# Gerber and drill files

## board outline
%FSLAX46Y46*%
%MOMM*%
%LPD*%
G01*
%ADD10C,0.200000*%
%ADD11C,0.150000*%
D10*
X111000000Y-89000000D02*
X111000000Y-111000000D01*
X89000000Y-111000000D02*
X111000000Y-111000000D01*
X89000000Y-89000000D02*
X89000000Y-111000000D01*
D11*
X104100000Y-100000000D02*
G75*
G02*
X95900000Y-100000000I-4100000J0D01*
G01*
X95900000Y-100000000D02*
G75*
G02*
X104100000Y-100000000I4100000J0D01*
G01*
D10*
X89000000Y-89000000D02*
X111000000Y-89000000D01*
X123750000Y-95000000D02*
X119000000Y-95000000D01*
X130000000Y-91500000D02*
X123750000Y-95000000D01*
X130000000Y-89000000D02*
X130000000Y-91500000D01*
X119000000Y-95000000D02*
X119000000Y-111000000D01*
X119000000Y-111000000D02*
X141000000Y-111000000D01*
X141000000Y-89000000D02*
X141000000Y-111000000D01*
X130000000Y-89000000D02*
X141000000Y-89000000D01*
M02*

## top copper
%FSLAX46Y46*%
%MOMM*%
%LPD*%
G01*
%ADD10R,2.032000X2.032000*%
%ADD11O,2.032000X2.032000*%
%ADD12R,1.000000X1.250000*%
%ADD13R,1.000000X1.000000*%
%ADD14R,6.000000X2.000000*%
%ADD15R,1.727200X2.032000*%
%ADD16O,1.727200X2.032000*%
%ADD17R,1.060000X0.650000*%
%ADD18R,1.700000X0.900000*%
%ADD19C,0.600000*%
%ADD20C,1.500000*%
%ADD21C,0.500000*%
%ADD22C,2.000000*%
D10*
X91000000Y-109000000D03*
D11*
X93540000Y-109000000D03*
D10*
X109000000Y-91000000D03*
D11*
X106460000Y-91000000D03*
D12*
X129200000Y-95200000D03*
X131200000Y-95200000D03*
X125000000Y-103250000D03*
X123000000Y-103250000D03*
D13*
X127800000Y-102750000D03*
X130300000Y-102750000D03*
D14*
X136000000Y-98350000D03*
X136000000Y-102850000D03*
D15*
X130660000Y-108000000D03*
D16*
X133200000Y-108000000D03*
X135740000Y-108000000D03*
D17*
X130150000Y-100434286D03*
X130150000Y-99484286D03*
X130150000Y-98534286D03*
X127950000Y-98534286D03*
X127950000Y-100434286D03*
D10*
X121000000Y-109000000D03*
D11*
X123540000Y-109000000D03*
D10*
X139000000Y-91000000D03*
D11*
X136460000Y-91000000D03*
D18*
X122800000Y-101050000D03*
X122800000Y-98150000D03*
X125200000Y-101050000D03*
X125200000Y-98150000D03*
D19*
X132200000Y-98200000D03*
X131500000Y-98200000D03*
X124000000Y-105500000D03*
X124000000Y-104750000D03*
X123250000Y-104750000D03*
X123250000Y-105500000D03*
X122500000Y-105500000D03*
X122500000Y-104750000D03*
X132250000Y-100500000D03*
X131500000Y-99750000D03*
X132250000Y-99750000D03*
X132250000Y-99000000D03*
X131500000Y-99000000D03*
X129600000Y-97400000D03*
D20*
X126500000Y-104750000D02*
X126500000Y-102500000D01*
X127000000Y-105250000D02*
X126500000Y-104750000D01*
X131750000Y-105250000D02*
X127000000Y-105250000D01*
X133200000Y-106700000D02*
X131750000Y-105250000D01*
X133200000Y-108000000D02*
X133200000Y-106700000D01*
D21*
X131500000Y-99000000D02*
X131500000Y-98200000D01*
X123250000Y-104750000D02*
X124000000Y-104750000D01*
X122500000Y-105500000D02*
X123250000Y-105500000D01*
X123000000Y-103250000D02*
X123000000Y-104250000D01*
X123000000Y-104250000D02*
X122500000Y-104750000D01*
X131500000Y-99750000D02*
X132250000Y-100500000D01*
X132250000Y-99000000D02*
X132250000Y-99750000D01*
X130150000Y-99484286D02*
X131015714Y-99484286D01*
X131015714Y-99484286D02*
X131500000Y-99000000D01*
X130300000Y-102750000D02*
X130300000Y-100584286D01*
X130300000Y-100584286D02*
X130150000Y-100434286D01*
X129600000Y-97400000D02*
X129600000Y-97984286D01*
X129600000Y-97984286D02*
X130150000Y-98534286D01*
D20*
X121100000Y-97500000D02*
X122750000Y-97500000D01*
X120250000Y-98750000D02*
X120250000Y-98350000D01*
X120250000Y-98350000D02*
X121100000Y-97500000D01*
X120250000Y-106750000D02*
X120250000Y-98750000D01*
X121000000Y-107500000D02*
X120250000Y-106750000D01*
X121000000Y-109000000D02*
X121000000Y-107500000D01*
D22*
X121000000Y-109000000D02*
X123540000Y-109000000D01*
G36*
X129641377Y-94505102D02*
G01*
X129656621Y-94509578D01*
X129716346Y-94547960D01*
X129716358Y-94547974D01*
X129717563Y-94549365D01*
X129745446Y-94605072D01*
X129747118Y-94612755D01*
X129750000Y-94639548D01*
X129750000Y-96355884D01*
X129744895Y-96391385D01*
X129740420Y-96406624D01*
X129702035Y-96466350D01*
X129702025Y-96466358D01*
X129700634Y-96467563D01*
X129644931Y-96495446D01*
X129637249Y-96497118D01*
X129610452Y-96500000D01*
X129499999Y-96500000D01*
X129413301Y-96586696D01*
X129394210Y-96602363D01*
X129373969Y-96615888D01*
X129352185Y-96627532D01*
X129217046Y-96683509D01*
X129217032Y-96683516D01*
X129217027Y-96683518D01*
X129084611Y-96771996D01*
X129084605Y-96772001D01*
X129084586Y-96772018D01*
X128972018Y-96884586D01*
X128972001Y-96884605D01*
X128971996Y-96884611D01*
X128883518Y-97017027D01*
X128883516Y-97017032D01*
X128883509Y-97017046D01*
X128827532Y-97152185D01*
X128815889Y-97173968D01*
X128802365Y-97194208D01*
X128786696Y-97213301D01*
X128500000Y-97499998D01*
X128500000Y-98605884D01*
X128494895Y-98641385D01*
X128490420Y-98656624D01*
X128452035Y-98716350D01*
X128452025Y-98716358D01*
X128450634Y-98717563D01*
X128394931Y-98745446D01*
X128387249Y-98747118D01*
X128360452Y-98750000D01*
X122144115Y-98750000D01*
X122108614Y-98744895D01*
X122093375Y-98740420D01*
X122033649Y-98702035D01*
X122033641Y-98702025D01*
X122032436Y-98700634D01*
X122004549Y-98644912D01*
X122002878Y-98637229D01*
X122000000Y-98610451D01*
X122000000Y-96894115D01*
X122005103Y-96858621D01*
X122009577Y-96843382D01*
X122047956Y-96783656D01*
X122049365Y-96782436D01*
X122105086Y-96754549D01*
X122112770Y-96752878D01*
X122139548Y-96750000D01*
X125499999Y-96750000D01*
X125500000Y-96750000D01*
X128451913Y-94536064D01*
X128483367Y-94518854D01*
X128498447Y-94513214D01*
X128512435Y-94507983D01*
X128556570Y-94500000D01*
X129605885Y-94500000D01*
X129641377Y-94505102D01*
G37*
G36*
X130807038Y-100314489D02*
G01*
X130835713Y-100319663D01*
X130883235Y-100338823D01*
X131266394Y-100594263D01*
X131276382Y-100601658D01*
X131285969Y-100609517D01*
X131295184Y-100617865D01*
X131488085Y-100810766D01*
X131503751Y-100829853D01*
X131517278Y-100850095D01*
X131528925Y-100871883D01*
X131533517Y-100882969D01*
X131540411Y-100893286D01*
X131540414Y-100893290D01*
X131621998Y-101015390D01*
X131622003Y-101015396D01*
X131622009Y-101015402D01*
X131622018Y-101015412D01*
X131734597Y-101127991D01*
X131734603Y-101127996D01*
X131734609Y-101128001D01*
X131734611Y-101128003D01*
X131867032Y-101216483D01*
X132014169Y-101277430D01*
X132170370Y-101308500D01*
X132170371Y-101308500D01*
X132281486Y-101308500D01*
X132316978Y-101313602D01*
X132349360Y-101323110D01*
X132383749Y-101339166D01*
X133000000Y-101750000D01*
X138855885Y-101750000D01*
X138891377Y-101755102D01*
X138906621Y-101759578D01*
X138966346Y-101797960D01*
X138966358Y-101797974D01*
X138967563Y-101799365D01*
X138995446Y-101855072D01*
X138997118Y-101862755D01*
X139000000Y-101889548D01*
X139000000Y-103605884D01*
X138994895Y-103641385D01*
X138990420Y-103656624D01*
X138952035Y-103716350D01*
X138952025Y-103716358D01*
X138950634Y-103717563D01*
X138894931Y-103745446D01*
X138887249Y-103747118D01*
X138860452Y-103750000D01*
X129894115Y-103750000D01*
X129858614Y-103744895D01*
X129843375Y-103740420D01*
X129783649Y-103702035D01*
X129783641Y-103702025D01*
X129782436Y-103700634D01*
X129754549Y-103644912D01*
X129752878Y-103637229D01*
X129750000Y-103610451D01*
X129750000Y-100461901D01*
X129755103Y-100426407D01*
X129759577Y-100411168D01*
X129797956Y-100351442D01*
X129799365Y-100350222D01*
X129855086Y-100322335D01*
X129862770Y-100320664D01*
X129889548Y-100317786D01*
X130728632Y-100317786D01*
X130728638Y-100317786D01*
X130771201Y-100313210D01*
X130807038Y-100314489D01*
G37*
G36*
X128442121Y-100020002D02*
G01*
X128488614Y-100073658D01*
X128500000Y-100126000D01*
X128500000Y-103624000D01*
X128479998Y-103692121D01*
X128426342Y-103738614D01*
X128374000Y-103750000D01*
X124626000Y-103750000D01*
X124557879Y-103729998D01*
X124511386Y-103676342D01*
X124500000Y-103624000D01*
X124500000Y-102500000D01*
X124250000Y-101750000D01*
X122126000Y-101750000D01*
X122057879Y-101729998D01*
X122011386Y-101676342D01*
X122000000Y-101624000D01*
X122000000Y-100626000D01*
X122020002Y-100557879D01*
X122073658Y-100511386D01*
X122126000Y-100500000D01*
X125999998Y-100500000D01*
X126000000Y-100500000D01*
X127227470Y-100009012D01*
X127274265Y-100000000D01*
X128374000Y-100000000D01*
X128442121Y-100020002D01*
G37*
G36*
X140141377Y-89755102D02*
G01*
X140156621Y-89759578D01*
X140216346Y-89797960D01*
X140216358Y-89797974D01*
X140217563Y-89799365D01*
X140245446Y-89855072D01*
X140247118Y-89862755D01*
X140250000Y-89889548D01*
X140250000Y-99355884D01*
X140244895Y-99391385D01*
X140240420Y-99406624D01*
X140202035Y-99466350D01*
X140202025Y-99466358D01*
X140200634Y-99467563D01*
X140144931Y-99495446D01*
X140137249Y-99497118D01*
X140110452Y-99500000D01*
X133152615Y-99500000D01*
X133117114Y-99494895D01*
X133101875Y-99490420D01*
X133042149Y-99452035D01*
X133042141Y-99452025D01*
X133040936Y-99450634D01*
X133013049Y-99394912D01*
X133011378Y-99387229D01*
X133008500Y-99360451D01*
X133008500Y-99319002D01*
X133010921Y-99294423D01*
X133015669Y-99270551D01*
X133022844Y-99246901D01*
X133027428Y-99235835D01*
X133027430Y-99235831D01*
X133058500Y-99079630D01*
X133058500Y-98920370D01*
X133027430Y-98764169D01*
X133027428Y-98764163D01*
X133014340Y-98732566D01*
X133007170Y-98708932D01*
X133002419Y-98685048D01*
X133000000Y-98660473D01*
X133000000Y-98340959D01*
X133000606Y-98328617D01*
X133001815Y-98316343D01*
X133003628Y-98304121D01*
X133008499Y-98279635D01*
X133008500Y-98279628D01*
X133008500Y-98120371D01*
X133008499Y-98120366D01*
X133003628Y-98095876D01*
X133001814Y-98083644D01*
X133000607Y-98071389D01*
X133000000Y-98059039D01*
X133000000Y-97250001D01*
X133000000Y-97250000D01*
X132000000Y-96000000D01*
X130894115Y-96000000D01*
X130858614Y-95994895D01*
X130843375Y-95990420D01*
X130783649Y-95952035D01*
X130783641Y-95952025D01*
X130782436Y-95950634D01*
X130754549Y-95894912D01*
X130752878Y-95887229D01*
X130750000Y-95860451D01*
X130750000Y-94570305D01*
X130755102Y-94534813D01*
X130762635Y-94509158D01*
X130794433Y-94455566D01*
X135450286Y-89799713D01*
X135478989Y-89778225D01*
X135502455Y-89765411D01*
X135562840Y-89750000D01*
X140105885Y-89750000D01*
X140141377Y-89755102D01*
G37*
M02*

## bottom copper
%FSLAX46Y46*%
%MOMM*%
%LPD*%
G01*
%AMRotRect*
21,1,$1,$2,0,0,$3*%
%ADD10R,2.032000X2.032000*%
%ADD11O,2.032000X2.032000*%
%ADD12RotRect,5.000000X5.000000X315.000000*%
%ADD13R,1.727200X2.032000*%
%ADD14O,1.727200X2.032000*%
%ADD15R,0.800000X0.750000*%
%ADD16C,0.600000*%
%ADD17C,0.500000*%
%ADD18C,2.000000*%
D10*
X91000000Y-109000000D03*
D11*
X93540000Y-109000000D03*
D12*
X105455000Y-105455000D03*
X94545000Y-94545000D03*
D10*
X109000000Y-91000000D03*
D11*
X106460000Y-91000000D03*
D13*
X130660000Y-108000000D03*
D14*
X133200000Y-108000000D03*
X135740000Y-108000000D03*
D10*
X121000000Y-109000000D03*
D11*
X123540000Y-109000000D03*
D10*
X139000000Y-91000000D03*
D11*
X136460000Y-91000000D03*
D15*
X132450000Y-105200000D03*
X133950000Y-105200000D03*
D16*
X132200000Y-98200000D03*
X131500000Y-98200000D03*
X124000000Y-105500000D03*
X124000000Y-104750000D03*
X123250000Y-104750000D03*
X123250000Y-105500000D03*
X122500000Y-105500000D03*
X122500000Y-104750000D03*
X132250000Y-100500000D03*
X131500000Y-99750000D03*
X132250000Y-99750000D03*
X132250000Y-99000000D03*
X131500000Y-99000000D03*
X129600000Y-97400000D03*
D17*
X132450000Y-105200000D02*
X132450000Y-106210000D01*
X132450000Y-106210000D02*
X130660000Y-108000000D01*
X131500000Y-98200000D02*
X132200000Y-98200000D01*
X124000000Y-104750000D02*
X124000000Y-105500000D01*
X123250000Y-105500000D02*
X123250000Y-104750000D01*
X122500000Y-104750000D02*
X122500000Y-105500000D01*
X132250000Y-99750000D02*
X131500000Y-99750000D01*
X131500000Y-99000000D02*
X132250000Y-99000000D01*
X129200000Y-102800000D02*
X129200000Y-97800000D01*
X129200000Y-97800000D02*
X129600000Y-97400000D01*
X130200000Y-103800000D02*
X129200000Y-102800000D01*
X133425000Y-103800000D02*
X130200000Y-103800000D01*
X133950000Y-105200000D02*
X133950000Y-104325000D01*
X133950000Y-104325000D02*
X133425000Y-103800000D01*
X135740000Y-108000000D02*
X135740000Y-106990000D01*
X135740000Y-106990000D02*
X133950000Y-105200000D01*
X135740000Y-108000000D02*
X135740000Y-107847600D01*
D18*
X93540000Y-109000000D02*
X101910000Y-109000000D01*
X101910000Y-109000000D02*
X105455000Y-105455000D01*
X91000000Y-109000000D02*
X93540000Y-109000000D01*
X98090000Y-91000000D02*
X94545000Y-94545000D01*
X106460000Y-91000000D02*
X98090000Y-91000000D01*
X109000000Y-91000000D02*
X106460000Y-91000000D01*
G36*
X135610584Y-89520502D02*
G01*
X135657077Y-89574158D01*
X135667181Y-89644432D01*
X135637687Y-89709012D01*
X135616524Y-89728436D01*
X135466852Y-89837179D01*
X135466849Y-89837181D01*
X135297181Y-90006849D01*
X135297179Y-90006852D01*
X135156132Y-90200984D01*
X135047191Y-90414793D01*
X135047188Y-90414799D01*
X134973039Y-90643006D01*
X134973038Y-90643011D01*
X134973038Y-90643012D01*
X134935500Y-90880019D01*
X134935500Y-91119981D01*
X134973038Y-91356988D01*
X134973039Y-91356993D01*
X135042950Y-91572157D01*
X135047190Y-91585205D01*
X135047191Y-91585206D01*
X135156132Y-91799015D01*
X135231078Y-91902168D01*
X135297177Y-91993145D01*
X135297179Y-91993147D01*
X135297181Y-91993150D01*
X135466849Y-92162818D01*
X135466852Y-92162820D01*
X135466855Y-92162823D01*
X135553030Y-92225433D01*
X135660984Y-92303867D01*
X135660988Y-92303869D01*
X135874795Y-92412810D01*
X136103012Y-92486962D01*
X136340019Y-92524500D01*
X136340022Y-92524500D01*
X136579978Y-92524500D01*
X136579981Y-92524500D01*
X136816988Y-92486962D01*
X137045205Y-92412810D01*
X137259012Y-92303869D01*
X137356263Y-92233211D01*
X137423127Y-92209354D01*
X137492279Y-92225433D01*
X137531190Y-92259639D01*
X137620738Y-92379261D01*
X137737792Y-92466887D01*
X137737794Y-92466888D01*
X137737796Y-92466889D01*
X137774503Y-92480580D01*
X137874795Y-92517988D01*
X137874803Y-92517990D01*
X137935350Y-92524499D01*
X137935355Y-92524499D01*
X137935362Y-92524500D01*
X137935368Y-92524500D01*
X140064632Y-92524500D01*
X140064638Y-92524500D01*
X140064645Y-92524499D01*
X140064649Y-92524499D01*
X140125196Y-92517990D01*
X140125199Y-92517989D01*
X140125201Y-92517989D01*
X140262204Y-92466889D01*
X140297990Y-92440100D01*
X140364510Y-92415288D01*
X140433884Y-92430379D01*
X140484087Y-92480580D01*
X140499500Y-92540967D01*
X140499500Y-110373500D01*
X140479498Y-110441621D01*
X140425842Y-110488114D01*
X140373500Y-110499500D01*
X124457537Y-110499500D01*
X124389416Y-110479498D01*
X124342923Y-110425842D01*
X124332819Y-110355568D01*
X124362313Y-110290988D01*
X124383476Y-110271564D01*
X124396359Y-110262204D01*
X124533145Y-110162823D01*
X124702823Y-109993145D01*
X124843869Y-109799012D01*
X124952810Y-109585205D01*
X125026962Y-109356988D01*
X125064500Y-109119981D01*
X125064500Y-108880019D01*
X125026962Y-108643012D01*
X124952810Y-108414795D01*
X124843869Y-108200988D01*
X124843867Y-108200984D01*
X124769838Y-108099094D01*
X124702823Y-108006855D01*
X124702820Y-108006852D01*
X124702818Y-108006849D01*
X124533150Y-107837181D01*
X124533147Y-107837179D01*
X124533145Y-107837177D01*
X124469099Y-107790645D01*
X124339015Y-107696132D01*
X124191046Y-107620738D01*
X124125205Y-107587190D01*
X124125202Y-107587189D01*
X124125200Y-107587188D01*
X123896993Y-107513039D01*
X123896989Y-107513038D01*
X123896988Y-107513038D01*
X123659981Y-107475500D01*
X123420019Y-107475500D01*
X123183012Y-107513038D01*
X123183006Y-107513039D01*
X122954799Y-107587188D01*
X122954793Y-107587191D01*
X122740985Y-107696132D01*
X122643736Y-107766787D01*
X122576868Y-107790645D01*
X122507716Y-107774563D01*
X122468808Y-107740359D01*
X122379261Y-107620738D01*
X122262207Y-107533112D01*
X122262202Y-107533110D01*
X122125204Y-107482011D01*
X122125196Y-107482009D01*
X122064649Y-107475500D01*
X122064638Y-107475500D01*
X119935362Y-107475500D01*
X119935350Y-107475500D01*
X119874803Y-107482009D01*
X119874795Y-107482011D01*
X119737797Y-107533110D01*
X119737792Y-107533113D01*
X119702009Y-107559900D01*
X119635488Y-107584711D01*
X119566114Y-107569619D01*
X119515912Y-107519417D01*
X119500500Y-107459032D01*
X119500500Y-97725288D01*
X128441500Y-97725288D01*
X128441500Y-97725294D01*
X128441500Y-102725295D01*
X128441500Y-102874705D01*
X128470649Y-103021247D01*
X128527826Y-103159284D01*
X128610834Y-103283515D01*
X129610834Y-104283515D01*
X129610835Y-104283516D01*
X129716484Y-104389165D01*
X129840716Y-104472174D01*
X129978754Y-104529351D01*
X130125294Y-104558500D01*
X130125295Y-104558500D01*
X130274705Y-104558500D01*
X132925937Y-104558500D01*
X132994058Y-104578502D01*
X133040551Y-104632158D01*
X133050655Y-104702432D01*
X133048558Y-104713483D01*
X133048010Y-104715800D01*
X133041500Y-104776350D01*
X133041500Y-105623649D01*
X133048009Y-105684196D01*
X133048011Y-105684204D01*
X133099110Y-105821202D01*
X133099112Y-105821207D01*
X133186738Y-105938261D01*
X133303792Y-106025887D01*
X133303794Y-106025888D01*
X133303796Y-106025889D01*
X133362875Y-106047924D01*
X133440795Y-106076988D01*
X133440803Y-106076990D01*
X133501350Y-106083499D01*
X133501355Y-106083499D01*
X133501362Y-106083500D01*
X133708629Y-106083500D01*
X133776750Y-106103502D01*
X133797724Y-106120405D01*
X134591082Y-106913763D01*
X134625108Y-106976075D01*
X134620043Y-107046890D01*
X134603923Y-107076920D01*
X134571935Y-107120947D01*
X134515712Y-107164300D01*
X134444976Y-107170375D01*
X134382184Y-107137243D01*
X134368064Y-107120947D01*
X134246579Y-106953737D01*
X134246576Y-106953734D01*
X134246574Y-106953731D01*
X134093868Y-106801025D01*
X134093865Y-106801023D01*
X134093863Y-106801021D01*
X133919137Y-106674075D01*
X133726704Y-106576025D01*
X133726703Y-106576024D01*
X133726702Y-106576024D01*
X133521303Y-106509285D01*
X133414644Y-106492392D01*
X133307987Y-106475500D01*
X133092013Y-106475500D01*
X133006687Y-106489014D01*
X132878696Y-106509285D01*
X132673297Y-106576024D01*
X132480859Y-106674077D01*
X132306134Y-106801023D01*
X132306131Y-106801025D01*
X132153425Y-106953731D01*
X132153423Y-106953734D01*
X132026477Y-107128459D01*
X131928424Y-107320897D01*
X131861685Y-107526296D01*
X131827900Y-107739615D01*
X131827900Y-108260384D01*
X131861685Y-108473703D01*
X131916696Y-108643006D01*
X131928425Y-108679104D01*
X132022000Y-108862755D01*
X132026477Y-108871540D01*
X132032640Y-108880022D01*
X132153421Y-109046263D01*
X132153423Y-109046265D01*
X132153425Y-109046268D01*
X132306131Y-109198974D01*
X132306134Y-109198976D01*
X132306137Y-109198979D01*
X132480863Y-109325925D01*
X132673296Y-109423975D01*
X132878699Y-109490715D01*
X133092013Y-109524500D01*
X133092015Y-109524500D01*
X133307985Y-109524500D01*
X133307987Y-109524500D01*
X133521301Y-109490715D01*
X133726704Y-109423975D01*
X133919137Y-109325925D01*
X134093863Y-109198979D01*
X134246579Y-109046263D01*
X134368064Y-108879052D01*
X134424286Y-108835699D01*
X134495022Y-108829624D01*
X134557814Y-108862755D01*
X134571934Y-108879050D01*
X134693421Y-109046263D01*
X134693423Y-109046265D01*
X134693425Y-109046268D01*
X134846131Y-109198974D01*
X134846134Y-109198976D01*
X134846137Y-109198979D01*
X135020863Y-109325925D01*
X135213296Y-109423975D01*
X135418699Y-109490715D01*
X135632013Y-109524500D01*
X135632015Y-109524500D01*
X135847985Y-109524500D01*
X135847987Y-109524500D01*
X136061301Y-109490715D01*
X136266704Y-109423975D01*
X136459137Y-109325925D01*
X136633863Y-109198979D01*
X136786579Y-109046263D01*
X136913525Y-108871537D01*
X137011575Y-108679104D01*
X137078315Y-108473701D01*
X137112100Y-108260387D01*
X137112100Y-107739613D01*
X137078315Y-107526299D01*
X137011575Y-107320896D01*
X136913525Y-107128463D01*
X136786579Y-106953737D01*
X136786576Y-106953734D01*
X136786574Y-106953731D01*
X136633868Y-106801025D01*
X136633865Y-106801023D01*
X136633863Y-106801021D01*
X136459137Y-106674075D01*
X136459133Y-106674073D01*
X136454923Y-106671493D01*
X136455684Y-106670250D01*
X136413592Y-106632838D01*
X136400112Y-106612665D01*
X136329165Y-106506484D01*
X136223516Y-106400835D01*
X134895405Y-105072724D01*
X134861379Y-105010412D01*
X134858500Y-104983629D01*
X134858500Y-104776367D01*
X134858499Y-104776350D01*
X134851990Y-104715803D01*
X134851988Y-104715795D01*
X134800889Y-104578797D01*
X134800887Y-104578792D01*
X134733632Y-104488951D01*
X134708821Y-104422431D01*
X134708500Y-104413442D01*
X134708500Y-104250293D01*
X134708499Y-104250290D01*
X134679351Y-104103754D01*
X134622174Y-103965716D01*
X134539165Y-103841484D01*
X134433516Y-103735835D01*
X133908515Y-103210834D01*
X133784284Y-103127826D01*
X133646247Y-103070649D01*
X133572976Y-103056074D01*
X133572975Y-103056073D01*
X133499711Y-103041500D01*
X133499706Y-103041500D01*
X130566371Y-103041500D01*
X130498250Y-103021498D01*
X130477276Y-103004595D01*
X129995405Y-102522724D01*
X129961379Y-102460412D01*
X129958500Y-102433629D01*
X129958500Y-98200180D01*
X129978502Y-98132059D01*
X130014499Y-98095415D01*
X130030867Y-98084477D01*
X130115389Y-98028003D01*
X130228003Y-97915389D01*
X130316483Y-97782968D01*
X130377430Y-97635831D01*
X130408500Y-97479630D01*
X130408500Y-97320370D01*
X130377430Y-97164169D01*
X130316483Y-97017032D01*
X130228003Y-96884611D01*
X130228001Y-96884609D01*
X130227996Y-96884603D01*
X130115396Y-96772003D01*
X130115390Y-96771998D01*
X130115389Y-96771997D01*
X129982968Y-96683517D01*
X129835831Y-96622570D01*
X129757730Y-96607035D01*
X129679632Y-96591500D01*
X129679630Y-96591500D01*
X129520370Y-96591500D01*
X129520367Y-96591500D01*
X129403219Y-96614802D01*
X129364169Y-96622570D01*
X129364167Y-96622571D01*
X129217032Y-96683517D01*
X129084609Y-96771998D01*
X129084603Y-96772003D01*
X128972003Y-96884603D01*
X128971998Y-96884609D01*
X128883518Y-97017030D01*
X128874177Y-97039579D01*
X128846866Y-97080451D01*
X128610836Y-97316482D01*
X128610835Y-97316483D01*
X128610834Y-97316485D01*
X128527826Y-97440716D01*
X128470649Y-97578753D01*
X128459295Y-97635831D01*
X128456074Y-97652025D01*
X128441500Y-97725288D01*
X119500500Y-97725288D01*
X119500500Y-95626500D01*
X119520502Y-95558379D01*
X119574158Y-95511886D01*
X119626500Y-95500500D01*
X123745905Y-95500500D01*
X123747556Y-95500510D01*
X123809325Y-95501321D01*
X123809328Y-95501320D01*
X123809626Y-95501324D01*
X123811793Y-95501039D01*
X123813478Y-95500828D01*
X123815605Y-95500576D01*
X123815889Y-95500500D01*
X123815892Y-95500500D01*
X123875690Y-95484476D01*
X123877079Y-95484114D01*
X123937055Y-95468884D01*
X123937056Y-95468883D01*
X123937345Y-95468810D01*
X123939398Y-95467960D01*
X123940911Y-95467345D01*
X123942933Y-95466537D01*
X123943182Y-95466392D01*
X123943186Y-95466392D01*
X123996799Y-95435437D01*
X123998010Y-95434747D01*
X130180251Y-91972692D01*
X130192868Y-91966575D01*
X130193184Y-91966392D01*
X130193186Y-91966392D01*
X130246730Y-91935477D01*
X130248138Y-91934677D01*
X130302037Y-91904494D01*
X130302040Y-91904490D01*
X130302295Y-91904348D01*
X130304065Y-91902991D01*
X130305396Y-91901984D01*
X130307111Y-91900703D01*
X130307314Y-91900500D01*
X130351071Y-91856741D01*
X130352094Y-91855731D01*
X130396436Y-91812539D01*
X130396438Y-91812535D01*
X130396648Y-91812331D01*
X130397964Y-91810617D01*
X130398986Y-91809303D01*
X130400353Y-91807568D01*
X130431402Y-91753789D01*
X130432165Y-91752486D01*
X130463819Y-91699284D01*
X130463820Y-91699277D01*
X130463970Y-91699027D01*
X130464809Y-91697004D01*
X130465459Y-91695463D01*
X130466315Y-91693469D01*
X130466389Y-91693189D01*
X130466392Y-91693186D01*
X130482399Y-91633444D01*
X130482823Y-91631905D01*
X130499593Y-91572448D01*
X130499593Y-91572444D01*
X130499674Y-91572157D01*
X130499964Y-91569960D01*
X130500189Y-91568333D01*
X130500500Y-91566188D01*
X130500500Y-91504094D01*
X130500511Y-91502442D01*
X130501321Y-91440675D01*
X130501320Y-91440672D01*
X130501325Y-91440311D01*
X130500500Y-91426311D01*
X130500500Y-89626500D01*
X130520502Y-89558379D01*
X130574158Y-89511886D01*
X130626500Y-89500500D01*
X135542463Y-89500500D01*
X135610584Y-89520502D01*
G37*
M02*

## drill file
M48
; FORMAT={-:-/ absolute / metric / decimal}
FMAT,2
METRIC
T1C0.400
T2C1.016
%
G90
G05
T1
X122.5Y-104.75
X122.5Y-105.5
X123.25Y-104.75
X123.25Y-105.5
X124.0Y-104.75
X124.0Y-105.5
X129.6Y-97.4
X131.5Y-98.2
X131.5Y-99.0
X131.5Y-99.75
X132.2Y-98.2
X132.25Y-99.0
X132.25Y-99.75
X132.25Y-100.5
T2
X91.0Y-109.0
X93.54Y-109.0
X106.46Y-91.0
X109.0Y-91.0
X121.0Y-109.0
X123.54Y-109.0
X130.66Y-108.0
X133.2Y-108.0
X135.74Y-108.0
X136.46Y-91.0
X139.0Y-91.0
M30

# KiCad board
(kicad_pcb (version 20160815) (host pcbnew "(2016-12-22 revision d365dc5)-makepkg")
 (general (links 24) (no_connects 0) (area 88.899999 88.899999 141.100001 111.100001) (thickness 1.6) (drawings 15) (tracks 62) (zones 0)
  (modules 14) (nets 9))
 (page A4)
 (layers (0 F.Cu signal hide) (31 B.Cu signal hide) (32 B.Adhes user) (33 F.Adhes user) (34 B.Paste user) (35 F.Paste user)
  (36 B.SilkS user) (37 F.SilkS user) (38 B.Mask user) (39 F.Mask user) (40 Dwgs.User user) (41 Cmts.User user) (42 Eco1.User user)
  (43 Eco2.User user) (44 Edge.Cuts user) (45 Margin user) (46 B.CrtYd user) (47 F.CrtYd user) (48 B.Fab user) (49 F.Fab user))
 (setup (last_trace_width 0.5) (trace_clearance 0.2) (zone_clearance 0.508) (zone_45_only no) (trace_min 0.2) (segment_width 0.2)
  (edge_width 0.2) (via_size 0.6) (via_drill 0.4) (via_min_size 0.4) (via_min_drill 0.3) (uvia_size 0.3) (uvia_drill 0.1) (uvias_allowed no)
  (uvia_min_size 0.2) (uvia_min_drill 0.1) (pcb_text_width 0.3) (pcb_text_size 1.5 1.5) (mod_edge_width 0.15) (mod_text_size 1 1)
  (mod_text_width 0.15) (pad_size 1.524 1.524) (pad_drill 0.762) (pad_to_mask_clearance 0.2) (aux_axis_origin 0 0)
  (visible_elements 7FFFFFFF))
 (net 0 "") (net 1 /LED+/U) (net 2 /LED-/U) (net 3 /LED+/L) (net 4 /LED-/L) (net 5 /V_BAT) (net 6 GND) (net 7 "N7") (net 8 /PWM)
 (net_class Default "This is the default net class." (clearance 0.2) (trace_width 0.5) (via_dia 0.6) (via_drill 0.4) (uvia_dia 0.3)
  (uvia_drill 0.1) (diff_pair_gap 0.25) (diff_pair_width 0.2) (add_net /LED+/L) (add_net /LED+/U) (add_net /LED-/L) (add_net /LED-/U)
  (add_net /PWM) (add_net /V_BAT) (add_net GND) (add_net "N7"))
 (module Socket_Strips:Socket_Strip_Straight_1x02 (layer B.Cu) (at 91 109)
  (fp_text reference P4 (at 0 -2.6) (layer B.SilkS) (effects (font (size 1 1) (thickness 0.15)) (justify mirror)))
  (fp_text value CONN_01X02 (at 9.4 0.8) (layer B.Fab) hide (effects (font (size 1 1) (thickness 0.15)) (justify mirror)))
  (pad 1 thru_hole rect (at 0 0) (size 2.032 2.032) (drill 1.016) (layers *.Cu *.Mask) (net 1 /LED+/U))
  (pad 2 thru_hole oval (at 2.54 0) (size 2.032 2.032) (drill 1.016) (layers *.Cu *.Mask) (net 1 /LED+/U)))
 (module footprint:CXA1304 (layer B.Cu) (at 100 100)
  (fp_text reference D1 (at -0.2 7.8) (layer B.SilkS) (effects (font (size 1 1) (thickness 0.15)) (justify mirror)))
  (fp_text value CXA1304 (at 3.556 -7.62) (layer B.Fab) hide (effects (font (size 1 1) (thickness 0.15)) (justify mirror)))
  (pad 2 smd rect (at 5.455 5.455 315) (size 5 5) (layers B.Cu B.Paste B.Mask) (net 1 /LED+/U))
  (pad 1 smd rect (at -5.455 -5.455 315) (size 5 5) (layers B.Cu B.Paste B.Mask) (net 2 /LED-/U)))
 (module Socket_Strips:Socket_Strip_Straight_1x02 (layer B.Cu) (at 109 91 180)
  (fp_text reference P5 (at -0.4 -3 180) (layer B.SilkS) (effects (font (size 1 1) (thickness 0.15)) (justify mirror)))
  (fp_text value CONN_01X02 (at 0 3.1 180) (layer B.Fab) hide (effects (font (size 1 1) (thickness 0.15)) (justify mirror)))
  (pad 1 thru_hole rect (at 0 0 180) (size 2.032 2.032) (drill 1.016) (layers *.Cu *.Mask) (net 2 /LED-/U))
  (pad 2 thru_hole oval (at 2.54 0 180) (size 2.032 2.032) (drill 1.016) (layers *.Cu *.Mask) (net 2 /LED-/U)))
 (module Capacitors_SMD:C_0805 (layer F.Cu) (at 130.2 95.2)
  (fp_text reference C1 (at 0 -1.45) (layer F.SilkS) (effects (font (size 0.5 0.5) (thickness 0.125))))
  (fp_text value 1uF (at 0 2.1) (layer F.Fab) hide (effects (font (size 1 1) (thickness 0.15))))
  (pad 1 smd rect (at -1 0) (size 1 1.25) (layers F.Cu F.Paste F.Mask) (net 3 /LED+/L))
  (pad 2 smd rect (at 1 0) (size 1 1.25) (layers F.Cu F.Paste F.Mask) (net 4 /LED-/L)))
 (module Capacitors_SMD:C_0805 (layer F.Cu) (at 124 103.25 180)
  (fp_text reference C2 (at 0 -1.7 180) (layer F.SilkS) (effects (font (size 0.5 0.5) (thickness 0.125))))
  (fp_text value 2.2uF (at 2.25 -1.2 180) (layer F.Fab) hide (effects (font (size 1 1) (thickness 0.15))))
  (pad 1 smd rect (at -1 0 180) (size 1 1.25) (layers F.Cu F.Paste F.Mask) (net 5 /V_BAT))
  (pad 2 smd rect (at 1 0 180) (size 1 1.25) (layers F.Cu F.Paste F.Mask) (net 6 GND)))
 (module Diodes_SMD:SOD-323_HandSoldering (layer F.Cu) (at 129.05 102.75)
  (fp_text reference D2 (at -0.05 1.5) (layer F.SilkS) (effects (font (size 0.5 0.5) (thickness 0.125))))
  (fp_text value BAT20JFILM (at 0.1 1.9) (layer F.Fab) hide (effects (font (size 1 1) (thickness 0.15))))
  (pad 1 smd rect (at -1.25 0) (size 1 1) (layers F.Cu F.Paste F.Mask) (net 5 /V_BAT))
  (pad 2 smd rect (at 1.25 0) (size 1 1) (layers F.Cu F.Paste F.Mask) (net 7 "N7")))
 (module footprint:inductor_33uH (layer F.Cu) (at 136 100.6 270)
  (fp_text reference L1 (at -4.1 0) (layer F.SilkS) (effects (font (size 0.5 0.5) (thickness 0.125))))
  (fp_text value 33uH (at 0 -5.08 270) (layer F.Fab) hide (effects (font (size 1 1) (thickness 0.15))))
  (pad 1 smd rect (at -2.25 0 270) (size 2 6) (layers F.Cu F.Paste F.Mask) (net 4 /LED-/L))
  (pad 2 smd rect (at 2.25 0 270) (size 2 6) (layers F.Cu F.Paste F.Mask) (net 7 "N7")))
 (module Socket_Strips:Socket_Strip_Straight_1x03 (layer B.Cu) (at 130.66 108)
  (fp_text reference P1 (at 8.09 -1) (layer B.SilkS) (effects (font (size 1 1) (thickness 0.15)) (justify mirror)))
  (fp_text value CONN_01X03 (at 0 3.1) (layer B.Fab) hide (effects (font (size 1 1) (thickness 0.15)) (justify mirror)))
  (pad 1 thru_hole rect (at 0 0) (size 1.7272 2.032) (drill 1.016) (layers *.Cu *.Mask) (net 6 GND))
  (pad 2 thru_hole oval (at 2.54 0) (size 1.7272 2.032) (drill 1.016) (layers *.Cu *.Mask) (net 5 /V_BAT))
  (pad 3 thru_hole oval (at 5.08 0) (size 1.7272 2.032) (drill 1.016) (layers *.Cu *.Mask) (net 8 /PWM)))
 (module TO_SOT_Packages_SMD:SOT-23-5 (layer F.Cu) (at 129.05 99.484286 180)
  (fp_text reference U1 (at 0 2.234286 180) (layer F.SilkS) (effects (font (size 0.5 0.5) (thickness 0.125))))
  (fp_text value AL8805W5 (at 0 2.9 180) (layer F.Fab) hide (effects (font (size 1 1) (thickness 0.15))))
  (pad 1 smd rect (at -1.1 -0.95 180) (size 1.06 0.65) (layers F.Cu F.Paste F.Mask) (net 7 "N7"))
  (pad 2 smd rect (at -1.1 0 180) (size 1.06 0.65) (layers F.Cu F.Paste F.Mask) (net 6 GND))
  (pad 3 smd rect (at -1.1 0.95 180) (size 1.06 0.65) (layers F.Cu F.Paste F.Mask) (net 8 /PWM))
  (pad 4 smd rect (at 1.1 0.95 180) (size 1.06 0.65) (layers F.Cu F.Paste F.Mask) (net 3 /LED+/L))
  (pad 5 smd rect (at 1.1 -0.95 180) (size 1.06 0.65) (layers F.Cu F.Paste F.Mask) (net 5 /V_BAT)))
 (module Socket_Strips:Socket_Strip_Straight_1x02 (layer F.Cu) (at 121 109)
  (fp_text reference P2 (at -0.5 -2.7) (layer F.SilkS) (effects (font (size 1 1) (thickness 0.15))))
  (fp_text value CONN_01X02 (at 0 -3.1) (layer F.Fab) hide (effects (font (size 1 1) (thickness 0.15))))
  (pad 1 thru_hole rect (at 0 0) (size 2.032 2.032) (drill 1.016) (layers *.Cu *.Mask) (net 3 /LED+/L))
  (pad 2 thru_hole oval (at 2.54 0) (size 2.032 2.032) (drill 1.016) (layers *.Cu *.Mask) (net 3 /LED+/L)))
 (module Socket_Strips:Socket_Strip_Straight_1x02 (layer F.Cu) (at 139 91 180)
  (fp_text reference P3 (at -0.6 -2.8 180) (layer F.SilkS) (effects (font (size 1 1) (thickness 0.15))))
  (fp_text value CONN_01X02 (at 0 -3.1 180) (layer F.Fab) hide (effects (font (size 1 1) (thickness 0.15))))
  (pad 1 thru_hole rect (at 0 0 180) (size 2.032 2.032) (drill 1.016) (layers *.Cu *.Mask) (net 4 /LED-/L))
  (pad 2 thru_hole oval (at 2.54 0 180) (size 2.032 2.032) (drill 1.016) (layers *.Cu *.Mask) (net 4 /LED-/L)))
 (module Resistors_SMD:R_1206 (layer F.Cu) (at 122.8 99.6 90)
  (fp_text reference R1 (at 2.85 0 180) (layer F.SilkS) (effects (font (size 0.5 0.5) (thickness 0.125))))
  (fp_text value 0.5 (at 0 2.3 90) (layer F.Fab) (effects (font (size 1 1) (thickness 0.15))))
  (pad 1 smd rect (at -1.45 0 90) (size 0.9 1.7) (layers F.Cu F.Paste F.Mask) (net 5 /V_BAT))
  (pad 2 smd rect (at 1.45 0 90) (size 0.9 1.7) (layers F.Cu F.Paste F.Mask) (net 3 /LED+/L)))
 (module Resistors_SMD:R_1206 (layer F.Cu) (at 125.2 99.6 90)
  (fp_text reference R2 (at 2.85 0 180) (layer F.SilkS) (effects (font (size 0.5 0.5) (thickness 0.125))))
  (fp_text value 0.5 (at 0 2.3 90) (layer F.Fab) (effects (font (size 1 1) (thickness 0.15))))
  (pad 1 smd rect (at -1.45 0 90) (size 0.9 1.7) (layers F.Cu F.Paste F.Mask) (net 5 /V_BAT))
  (pad 2 smd rect (at 1.45 0 90) (size 0.9 1.7) (layers F.Cu F.Paste F.Mask) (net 3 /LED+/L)))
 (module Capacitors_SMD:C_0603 (layer B.Cu) (at 133.2 105.2 180)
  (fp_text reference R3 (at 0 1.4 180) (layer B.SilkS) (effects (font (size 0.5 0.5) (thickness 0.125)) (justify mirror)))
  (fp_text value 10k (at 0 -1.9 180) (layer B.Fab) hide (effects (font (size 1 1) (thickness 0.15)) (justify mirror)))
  (pad 2 smd rect (at 0.75 0 180) (size 0.8 0.75) (layers B.Cu B.Paste B.Mask) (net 6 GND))
  (pad 1 smd rect (at -0.75 0 180) (size 0.8 0.75) (layers B.Cu B.Paste B.Mask) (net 8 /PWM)))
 (gr_line (start 111 89) (end 111 111) (layer Edge.Cuts) (width 0.2))
 (gr_line (start 89 111) (end 111 111) (layer Edge.Cuts) (width 0.2))
 (gr_line (start 89 89) (end 89 111) (layer Edge.Cuts) (width 0.2))
 (gr_circle (center 100 100) (end 100 95.9) (layer Edge.Cuts) (width 0.15))
 (gr_line (start 89 89) (end 111 89) (layer Edge.Cuts) (width 0.2))
 (gr_line (start 123.75 95) (end 119 95) (layer Edge.Cuts) (width 0.2))
 (gr_line (start 130 91.5) (end 123.75 95) (layer Edge.Cuts) (width 0.2))
 (gr_line (start 130 89) (end 130 91.5) (layer Edge.Cuts) (width 0.2))
 (gr_line (start 119 95) (end 119 111) (layer Edge.Cuts) (width 0.2))
 (gr_line (start 119 111) (end 141 111) (layer Edge.Cuts) (width 0.2))
 (gr_line (start 141 89) (end 141 111) (layer Edge.Cuts) (width 0.2))
 (gr_line (start 130 89) (end 141 89) (layer Edge.Cuts) (width 0.2))
 (segment (start 126.5 104.75) (end 126.5 102.5) (width 1.5) (layer F.Cu) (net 5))
 (segment (start 127 105.25) (end 126.5 104.75) (width 1.5) (layer F.Cu) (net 5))
 (segment (start 131.75 105.25) (end 127 105.25) (width 1.5) (layer F.Cu) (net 5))
 (segment (start 133.2 106.7) (end 131.75 105.25) (width 1.5) (layer F.Cu) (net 5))
 (segment (start 133.2 108) (end 133.2 106.7) (width 1.5) (layer F.Cu) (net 5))
 (segment (start 132.45 105.2) (end 132.45 106.21) (width 0.5) (layer B.Cu) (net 6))
 (segment (start 132.45 106.21) (end 130.66 108) (width 0.5) (layer B.Cu) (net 6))
 (segment (start 131.5 98.2) (end 132.2 98.2) (width 0.5) (layer B.Cu) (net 6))
 (via (at 132.2 98.2) (size 0.6) (drill 0.4) (layers F.Cu B.Cu) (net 6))
 (segment (start 131.5 99) (end 131.5 98.2) (width 0.5) (layer F.Cu) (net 6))
 (via (at 131.5 98.2) (size 0.6) (drill 0.4) (layers F.Cu B.Cu) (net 6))
 (segment (start 124 104.75) (end 124 105.5) (width 0.5) (layer B.Cu) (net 6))
 (via (at 124 105.5) (size 0.6) (drill 0.4) (layers F.Cu B.Cu) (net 6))
 (segment (start 123.25 104.75) (end 124 104.75) (width 0.5) (layer F.Cu) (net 6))
 (via (at 124 104.75) (size 0.6) (drill 0.4) (layers F.Cu B.Cu) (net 6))
 (segment (start 123.25 105.5) (end 123.25 104.75) (width 0.5) (layer B.Cu) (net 6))
 (via (at 123.25 104.75) (size 0.6) (drill 0.4) (layers F.Cu B.Cu) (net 6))
 (segment (start 122.5 105.5) (end 123.25 105.5) (width 0.5) (layer F.Cu) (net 6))
 (via (at 123.25 105.5) (size 0.6) (drill 0.4) (layers F.Cu B.Cu) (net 6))
 (segment (start 122.5 104.75) (end 122.5 105.5) (width 0.5) (layer B.Cu) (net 6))
 (via (at 122.5 105.5) (size 0.6) (drill 0.4) (layers F.Cu B.Cu) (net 6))
 (segment (start 123 103.25) (end 123 104.25) (width 0.5) (layer F.Cu) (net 6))
 (segment (start 123 104.25) (end 122.5 104.75) (width 0.5) (layer F.Cu) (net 6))
 (via (at 122.5 104.75) (size 0.6) (drill 0.4) (layers F.Cu B.Cu) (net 6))
 (segment (start 131.5 99.75) (end 132.25 100.5) (width 0.5) (layer F.Cu) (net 6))
 (via (at 132.25 100.5) (size 0.6) (drill 0.4) (layers F.Cu B.Cu) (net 6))
 (segment (start 132.25 99.75) (end 131.5 99.75) (width 0.5) (layer B.Cu) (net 6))
 (via (at 131.5 99.75) (size 0.6) (drill 0.4) (layers F.Cu B.Cu) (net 6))
 (segment (start 132.25 99) (end 132.25 99.75) (width 0.5) (layer F.Cu) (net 6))
 (via (at 132.25 99.75) (size 0.6) (drill 0.4) (layers F.Cu B.Cu) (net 6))
 (segment (start 131.5 99) (end 132.25 99) (width 0.5) (layer B.Cu) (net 6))
 (via (at 132.25 99) (size 0.6) (drill 0.4) (layers F.Cu B.Cu) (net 6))
 (segment (start 130.15 99.484286) (end 131.015714 99.484286) (width 0.5) (layer F.Cu) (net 6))
 (segment (start 131.015714 99.484286) (end 131.5 99) (width 0.5) (layer F.Cu) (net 6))
 (via (at 131.5 99) (size 0.6) (drill 0.4) (layers F.Cu B.Cu) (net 6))
 (segment (start 130.3 102.75) (end 130.3 100.584286) (width 0.5) (layer F.Cu) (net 7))
 (segment (start 130.3 100.584286) (end 130.15 100.434286) (width 0.5) (layer F.Cu) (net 7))
 (segment (start 129.6 97.4) (end 129.6 97.984286) (width 0.5) (layer F.Cu) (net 8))
 (segment (start 129.6 97.984286) (end 130.15 98.534286) (width 0.5) (layer F.Cu) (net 8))
 (segment (start 129.2 102.8) (end 129.2 97.8) (width 0.5) (layer B.Cu) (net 8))
 (segment (start 129.2 97.8) (end 129.6 97.4) (width 0.5) (layer B.Cu) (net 8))
 (via (at 129.6 97.4) (size 0.6) (drill 0.4) (layers F.Cu B.Cu) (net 8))
 (segment (start 130.2 103.8) (end 129.2 102.8) (width 0.5) (layer B.Cu) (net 8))
 (segment (start 133.425 103.8) (end 130.2 103.8) (width 0.5) (layer B.Cu) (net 8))
 (segment (start 133.95 105.2) (end 133.95 104.325) (width 0.5) (layer B.Cu) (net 8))
 (segment (start 133.95 104.325) (end 133.425 103.8) (width 0.5) (layer B.Cu) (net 8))
 (segment (start 135.74 108) (end 135.74 106.99) (width 0.5) (layer B.Cu) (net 8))
 (segment (start 135.74 106.99) (end 133.95 105.2) (width 0.5) (layer B.Cu) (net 8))
 (segment (start 135.74 108) (end 135.74 107.8476) (width 0.5) (layer B.Cu) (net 8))
 (segment (start 121.1 97.5) (end 122.75 97.5) (width 1.5) (layer F.Cu) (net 3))
 (segment (start 120.25 98.75) (end 120.25 98.35) (width 1.5) (layer F.Cu) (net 3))
 (segment (start 120.25 98.35) (end 121.1 97.5) (width 1.5) (layer F.Cu) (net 3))
 (segment (start 120.25 106.75) (end 120.25 98.75) (width 1.5) (layer F.Cu) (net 3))
 (segment (start 121 107.5) (end 120.25 106.75) (width 1.5) (layer F.Cu) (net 3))
 (segment (start 121 109) (end 121 107.5) (width 1.5) (layer F.Cu) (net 3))
 (segment (start 121 109) (end 123.54 109) (width 2) (layer F.Cu) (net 3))
 (segment (start 93.54 109) (end 101.91 109) (width 2) (layer B.Cu) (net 1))
 (segment (start 101.91 109) (end 105.455 105.455) (width 2) (layer B.Cu) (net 1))
 (segment (start 91 109) (end 93.54 109) (width 2) (layer B.Cu) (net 1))
 (segment (start 98.09 91) (end 94.545 94.545) (width 2) (layer B.Cu) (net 2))
 (segment (start 106.46 91) (end 98.09 91) (width 2) (layer B.Cu) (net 2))
 (segment (start 109 91) (end 106.46 91) (width 2) (layer B.Cu) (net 2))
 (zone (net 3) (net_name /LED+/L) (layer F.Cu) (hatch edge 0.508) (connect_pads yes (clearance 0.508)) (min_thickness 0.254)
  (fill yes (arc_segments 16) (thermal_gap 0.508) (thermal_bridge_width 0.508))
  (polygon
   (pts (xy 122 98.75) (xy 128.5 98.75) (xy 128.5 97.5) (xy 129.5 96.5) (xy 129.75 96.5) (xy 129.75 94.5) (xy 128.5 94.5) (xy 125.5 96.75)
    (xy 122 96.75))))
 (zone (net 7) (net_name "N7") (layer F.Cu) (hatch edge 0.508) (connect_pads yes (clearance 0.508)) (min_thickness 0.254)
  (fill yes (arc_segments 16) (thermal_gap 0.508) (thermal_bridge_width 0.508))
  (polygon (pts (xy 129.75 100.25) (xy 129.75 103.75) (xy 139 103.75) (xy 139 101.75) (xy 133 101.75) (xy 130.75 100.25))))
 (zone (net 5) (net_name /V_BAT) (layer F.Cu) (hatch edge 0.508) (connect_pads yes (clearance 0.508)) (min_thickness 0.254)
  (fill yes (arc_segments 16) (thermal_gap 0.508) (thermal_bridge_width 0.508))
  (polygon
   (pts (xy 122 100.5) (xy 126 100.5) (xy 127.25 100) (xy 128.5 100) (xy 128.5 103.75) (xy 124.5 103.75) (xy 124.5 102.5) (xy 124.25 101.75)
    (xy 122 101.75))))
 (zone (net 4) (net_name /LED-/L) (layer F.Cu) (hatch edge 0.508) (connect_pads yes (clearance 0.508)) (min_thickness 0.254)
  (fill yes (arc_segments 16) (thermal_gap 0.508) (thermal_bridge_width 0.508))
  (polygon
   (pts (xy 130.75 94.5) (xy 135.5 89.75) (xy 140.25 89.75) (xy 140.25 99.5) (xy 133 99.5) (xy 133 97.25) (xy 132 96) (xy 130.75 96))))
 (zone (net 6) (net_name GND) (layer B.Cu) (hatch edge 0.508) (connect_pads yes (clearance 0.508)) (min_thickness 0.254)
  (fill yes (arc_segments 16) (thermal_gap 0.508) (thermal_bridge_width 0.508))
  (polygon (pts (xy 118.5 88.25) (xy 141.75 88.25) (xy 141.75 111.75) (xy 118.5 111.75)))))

